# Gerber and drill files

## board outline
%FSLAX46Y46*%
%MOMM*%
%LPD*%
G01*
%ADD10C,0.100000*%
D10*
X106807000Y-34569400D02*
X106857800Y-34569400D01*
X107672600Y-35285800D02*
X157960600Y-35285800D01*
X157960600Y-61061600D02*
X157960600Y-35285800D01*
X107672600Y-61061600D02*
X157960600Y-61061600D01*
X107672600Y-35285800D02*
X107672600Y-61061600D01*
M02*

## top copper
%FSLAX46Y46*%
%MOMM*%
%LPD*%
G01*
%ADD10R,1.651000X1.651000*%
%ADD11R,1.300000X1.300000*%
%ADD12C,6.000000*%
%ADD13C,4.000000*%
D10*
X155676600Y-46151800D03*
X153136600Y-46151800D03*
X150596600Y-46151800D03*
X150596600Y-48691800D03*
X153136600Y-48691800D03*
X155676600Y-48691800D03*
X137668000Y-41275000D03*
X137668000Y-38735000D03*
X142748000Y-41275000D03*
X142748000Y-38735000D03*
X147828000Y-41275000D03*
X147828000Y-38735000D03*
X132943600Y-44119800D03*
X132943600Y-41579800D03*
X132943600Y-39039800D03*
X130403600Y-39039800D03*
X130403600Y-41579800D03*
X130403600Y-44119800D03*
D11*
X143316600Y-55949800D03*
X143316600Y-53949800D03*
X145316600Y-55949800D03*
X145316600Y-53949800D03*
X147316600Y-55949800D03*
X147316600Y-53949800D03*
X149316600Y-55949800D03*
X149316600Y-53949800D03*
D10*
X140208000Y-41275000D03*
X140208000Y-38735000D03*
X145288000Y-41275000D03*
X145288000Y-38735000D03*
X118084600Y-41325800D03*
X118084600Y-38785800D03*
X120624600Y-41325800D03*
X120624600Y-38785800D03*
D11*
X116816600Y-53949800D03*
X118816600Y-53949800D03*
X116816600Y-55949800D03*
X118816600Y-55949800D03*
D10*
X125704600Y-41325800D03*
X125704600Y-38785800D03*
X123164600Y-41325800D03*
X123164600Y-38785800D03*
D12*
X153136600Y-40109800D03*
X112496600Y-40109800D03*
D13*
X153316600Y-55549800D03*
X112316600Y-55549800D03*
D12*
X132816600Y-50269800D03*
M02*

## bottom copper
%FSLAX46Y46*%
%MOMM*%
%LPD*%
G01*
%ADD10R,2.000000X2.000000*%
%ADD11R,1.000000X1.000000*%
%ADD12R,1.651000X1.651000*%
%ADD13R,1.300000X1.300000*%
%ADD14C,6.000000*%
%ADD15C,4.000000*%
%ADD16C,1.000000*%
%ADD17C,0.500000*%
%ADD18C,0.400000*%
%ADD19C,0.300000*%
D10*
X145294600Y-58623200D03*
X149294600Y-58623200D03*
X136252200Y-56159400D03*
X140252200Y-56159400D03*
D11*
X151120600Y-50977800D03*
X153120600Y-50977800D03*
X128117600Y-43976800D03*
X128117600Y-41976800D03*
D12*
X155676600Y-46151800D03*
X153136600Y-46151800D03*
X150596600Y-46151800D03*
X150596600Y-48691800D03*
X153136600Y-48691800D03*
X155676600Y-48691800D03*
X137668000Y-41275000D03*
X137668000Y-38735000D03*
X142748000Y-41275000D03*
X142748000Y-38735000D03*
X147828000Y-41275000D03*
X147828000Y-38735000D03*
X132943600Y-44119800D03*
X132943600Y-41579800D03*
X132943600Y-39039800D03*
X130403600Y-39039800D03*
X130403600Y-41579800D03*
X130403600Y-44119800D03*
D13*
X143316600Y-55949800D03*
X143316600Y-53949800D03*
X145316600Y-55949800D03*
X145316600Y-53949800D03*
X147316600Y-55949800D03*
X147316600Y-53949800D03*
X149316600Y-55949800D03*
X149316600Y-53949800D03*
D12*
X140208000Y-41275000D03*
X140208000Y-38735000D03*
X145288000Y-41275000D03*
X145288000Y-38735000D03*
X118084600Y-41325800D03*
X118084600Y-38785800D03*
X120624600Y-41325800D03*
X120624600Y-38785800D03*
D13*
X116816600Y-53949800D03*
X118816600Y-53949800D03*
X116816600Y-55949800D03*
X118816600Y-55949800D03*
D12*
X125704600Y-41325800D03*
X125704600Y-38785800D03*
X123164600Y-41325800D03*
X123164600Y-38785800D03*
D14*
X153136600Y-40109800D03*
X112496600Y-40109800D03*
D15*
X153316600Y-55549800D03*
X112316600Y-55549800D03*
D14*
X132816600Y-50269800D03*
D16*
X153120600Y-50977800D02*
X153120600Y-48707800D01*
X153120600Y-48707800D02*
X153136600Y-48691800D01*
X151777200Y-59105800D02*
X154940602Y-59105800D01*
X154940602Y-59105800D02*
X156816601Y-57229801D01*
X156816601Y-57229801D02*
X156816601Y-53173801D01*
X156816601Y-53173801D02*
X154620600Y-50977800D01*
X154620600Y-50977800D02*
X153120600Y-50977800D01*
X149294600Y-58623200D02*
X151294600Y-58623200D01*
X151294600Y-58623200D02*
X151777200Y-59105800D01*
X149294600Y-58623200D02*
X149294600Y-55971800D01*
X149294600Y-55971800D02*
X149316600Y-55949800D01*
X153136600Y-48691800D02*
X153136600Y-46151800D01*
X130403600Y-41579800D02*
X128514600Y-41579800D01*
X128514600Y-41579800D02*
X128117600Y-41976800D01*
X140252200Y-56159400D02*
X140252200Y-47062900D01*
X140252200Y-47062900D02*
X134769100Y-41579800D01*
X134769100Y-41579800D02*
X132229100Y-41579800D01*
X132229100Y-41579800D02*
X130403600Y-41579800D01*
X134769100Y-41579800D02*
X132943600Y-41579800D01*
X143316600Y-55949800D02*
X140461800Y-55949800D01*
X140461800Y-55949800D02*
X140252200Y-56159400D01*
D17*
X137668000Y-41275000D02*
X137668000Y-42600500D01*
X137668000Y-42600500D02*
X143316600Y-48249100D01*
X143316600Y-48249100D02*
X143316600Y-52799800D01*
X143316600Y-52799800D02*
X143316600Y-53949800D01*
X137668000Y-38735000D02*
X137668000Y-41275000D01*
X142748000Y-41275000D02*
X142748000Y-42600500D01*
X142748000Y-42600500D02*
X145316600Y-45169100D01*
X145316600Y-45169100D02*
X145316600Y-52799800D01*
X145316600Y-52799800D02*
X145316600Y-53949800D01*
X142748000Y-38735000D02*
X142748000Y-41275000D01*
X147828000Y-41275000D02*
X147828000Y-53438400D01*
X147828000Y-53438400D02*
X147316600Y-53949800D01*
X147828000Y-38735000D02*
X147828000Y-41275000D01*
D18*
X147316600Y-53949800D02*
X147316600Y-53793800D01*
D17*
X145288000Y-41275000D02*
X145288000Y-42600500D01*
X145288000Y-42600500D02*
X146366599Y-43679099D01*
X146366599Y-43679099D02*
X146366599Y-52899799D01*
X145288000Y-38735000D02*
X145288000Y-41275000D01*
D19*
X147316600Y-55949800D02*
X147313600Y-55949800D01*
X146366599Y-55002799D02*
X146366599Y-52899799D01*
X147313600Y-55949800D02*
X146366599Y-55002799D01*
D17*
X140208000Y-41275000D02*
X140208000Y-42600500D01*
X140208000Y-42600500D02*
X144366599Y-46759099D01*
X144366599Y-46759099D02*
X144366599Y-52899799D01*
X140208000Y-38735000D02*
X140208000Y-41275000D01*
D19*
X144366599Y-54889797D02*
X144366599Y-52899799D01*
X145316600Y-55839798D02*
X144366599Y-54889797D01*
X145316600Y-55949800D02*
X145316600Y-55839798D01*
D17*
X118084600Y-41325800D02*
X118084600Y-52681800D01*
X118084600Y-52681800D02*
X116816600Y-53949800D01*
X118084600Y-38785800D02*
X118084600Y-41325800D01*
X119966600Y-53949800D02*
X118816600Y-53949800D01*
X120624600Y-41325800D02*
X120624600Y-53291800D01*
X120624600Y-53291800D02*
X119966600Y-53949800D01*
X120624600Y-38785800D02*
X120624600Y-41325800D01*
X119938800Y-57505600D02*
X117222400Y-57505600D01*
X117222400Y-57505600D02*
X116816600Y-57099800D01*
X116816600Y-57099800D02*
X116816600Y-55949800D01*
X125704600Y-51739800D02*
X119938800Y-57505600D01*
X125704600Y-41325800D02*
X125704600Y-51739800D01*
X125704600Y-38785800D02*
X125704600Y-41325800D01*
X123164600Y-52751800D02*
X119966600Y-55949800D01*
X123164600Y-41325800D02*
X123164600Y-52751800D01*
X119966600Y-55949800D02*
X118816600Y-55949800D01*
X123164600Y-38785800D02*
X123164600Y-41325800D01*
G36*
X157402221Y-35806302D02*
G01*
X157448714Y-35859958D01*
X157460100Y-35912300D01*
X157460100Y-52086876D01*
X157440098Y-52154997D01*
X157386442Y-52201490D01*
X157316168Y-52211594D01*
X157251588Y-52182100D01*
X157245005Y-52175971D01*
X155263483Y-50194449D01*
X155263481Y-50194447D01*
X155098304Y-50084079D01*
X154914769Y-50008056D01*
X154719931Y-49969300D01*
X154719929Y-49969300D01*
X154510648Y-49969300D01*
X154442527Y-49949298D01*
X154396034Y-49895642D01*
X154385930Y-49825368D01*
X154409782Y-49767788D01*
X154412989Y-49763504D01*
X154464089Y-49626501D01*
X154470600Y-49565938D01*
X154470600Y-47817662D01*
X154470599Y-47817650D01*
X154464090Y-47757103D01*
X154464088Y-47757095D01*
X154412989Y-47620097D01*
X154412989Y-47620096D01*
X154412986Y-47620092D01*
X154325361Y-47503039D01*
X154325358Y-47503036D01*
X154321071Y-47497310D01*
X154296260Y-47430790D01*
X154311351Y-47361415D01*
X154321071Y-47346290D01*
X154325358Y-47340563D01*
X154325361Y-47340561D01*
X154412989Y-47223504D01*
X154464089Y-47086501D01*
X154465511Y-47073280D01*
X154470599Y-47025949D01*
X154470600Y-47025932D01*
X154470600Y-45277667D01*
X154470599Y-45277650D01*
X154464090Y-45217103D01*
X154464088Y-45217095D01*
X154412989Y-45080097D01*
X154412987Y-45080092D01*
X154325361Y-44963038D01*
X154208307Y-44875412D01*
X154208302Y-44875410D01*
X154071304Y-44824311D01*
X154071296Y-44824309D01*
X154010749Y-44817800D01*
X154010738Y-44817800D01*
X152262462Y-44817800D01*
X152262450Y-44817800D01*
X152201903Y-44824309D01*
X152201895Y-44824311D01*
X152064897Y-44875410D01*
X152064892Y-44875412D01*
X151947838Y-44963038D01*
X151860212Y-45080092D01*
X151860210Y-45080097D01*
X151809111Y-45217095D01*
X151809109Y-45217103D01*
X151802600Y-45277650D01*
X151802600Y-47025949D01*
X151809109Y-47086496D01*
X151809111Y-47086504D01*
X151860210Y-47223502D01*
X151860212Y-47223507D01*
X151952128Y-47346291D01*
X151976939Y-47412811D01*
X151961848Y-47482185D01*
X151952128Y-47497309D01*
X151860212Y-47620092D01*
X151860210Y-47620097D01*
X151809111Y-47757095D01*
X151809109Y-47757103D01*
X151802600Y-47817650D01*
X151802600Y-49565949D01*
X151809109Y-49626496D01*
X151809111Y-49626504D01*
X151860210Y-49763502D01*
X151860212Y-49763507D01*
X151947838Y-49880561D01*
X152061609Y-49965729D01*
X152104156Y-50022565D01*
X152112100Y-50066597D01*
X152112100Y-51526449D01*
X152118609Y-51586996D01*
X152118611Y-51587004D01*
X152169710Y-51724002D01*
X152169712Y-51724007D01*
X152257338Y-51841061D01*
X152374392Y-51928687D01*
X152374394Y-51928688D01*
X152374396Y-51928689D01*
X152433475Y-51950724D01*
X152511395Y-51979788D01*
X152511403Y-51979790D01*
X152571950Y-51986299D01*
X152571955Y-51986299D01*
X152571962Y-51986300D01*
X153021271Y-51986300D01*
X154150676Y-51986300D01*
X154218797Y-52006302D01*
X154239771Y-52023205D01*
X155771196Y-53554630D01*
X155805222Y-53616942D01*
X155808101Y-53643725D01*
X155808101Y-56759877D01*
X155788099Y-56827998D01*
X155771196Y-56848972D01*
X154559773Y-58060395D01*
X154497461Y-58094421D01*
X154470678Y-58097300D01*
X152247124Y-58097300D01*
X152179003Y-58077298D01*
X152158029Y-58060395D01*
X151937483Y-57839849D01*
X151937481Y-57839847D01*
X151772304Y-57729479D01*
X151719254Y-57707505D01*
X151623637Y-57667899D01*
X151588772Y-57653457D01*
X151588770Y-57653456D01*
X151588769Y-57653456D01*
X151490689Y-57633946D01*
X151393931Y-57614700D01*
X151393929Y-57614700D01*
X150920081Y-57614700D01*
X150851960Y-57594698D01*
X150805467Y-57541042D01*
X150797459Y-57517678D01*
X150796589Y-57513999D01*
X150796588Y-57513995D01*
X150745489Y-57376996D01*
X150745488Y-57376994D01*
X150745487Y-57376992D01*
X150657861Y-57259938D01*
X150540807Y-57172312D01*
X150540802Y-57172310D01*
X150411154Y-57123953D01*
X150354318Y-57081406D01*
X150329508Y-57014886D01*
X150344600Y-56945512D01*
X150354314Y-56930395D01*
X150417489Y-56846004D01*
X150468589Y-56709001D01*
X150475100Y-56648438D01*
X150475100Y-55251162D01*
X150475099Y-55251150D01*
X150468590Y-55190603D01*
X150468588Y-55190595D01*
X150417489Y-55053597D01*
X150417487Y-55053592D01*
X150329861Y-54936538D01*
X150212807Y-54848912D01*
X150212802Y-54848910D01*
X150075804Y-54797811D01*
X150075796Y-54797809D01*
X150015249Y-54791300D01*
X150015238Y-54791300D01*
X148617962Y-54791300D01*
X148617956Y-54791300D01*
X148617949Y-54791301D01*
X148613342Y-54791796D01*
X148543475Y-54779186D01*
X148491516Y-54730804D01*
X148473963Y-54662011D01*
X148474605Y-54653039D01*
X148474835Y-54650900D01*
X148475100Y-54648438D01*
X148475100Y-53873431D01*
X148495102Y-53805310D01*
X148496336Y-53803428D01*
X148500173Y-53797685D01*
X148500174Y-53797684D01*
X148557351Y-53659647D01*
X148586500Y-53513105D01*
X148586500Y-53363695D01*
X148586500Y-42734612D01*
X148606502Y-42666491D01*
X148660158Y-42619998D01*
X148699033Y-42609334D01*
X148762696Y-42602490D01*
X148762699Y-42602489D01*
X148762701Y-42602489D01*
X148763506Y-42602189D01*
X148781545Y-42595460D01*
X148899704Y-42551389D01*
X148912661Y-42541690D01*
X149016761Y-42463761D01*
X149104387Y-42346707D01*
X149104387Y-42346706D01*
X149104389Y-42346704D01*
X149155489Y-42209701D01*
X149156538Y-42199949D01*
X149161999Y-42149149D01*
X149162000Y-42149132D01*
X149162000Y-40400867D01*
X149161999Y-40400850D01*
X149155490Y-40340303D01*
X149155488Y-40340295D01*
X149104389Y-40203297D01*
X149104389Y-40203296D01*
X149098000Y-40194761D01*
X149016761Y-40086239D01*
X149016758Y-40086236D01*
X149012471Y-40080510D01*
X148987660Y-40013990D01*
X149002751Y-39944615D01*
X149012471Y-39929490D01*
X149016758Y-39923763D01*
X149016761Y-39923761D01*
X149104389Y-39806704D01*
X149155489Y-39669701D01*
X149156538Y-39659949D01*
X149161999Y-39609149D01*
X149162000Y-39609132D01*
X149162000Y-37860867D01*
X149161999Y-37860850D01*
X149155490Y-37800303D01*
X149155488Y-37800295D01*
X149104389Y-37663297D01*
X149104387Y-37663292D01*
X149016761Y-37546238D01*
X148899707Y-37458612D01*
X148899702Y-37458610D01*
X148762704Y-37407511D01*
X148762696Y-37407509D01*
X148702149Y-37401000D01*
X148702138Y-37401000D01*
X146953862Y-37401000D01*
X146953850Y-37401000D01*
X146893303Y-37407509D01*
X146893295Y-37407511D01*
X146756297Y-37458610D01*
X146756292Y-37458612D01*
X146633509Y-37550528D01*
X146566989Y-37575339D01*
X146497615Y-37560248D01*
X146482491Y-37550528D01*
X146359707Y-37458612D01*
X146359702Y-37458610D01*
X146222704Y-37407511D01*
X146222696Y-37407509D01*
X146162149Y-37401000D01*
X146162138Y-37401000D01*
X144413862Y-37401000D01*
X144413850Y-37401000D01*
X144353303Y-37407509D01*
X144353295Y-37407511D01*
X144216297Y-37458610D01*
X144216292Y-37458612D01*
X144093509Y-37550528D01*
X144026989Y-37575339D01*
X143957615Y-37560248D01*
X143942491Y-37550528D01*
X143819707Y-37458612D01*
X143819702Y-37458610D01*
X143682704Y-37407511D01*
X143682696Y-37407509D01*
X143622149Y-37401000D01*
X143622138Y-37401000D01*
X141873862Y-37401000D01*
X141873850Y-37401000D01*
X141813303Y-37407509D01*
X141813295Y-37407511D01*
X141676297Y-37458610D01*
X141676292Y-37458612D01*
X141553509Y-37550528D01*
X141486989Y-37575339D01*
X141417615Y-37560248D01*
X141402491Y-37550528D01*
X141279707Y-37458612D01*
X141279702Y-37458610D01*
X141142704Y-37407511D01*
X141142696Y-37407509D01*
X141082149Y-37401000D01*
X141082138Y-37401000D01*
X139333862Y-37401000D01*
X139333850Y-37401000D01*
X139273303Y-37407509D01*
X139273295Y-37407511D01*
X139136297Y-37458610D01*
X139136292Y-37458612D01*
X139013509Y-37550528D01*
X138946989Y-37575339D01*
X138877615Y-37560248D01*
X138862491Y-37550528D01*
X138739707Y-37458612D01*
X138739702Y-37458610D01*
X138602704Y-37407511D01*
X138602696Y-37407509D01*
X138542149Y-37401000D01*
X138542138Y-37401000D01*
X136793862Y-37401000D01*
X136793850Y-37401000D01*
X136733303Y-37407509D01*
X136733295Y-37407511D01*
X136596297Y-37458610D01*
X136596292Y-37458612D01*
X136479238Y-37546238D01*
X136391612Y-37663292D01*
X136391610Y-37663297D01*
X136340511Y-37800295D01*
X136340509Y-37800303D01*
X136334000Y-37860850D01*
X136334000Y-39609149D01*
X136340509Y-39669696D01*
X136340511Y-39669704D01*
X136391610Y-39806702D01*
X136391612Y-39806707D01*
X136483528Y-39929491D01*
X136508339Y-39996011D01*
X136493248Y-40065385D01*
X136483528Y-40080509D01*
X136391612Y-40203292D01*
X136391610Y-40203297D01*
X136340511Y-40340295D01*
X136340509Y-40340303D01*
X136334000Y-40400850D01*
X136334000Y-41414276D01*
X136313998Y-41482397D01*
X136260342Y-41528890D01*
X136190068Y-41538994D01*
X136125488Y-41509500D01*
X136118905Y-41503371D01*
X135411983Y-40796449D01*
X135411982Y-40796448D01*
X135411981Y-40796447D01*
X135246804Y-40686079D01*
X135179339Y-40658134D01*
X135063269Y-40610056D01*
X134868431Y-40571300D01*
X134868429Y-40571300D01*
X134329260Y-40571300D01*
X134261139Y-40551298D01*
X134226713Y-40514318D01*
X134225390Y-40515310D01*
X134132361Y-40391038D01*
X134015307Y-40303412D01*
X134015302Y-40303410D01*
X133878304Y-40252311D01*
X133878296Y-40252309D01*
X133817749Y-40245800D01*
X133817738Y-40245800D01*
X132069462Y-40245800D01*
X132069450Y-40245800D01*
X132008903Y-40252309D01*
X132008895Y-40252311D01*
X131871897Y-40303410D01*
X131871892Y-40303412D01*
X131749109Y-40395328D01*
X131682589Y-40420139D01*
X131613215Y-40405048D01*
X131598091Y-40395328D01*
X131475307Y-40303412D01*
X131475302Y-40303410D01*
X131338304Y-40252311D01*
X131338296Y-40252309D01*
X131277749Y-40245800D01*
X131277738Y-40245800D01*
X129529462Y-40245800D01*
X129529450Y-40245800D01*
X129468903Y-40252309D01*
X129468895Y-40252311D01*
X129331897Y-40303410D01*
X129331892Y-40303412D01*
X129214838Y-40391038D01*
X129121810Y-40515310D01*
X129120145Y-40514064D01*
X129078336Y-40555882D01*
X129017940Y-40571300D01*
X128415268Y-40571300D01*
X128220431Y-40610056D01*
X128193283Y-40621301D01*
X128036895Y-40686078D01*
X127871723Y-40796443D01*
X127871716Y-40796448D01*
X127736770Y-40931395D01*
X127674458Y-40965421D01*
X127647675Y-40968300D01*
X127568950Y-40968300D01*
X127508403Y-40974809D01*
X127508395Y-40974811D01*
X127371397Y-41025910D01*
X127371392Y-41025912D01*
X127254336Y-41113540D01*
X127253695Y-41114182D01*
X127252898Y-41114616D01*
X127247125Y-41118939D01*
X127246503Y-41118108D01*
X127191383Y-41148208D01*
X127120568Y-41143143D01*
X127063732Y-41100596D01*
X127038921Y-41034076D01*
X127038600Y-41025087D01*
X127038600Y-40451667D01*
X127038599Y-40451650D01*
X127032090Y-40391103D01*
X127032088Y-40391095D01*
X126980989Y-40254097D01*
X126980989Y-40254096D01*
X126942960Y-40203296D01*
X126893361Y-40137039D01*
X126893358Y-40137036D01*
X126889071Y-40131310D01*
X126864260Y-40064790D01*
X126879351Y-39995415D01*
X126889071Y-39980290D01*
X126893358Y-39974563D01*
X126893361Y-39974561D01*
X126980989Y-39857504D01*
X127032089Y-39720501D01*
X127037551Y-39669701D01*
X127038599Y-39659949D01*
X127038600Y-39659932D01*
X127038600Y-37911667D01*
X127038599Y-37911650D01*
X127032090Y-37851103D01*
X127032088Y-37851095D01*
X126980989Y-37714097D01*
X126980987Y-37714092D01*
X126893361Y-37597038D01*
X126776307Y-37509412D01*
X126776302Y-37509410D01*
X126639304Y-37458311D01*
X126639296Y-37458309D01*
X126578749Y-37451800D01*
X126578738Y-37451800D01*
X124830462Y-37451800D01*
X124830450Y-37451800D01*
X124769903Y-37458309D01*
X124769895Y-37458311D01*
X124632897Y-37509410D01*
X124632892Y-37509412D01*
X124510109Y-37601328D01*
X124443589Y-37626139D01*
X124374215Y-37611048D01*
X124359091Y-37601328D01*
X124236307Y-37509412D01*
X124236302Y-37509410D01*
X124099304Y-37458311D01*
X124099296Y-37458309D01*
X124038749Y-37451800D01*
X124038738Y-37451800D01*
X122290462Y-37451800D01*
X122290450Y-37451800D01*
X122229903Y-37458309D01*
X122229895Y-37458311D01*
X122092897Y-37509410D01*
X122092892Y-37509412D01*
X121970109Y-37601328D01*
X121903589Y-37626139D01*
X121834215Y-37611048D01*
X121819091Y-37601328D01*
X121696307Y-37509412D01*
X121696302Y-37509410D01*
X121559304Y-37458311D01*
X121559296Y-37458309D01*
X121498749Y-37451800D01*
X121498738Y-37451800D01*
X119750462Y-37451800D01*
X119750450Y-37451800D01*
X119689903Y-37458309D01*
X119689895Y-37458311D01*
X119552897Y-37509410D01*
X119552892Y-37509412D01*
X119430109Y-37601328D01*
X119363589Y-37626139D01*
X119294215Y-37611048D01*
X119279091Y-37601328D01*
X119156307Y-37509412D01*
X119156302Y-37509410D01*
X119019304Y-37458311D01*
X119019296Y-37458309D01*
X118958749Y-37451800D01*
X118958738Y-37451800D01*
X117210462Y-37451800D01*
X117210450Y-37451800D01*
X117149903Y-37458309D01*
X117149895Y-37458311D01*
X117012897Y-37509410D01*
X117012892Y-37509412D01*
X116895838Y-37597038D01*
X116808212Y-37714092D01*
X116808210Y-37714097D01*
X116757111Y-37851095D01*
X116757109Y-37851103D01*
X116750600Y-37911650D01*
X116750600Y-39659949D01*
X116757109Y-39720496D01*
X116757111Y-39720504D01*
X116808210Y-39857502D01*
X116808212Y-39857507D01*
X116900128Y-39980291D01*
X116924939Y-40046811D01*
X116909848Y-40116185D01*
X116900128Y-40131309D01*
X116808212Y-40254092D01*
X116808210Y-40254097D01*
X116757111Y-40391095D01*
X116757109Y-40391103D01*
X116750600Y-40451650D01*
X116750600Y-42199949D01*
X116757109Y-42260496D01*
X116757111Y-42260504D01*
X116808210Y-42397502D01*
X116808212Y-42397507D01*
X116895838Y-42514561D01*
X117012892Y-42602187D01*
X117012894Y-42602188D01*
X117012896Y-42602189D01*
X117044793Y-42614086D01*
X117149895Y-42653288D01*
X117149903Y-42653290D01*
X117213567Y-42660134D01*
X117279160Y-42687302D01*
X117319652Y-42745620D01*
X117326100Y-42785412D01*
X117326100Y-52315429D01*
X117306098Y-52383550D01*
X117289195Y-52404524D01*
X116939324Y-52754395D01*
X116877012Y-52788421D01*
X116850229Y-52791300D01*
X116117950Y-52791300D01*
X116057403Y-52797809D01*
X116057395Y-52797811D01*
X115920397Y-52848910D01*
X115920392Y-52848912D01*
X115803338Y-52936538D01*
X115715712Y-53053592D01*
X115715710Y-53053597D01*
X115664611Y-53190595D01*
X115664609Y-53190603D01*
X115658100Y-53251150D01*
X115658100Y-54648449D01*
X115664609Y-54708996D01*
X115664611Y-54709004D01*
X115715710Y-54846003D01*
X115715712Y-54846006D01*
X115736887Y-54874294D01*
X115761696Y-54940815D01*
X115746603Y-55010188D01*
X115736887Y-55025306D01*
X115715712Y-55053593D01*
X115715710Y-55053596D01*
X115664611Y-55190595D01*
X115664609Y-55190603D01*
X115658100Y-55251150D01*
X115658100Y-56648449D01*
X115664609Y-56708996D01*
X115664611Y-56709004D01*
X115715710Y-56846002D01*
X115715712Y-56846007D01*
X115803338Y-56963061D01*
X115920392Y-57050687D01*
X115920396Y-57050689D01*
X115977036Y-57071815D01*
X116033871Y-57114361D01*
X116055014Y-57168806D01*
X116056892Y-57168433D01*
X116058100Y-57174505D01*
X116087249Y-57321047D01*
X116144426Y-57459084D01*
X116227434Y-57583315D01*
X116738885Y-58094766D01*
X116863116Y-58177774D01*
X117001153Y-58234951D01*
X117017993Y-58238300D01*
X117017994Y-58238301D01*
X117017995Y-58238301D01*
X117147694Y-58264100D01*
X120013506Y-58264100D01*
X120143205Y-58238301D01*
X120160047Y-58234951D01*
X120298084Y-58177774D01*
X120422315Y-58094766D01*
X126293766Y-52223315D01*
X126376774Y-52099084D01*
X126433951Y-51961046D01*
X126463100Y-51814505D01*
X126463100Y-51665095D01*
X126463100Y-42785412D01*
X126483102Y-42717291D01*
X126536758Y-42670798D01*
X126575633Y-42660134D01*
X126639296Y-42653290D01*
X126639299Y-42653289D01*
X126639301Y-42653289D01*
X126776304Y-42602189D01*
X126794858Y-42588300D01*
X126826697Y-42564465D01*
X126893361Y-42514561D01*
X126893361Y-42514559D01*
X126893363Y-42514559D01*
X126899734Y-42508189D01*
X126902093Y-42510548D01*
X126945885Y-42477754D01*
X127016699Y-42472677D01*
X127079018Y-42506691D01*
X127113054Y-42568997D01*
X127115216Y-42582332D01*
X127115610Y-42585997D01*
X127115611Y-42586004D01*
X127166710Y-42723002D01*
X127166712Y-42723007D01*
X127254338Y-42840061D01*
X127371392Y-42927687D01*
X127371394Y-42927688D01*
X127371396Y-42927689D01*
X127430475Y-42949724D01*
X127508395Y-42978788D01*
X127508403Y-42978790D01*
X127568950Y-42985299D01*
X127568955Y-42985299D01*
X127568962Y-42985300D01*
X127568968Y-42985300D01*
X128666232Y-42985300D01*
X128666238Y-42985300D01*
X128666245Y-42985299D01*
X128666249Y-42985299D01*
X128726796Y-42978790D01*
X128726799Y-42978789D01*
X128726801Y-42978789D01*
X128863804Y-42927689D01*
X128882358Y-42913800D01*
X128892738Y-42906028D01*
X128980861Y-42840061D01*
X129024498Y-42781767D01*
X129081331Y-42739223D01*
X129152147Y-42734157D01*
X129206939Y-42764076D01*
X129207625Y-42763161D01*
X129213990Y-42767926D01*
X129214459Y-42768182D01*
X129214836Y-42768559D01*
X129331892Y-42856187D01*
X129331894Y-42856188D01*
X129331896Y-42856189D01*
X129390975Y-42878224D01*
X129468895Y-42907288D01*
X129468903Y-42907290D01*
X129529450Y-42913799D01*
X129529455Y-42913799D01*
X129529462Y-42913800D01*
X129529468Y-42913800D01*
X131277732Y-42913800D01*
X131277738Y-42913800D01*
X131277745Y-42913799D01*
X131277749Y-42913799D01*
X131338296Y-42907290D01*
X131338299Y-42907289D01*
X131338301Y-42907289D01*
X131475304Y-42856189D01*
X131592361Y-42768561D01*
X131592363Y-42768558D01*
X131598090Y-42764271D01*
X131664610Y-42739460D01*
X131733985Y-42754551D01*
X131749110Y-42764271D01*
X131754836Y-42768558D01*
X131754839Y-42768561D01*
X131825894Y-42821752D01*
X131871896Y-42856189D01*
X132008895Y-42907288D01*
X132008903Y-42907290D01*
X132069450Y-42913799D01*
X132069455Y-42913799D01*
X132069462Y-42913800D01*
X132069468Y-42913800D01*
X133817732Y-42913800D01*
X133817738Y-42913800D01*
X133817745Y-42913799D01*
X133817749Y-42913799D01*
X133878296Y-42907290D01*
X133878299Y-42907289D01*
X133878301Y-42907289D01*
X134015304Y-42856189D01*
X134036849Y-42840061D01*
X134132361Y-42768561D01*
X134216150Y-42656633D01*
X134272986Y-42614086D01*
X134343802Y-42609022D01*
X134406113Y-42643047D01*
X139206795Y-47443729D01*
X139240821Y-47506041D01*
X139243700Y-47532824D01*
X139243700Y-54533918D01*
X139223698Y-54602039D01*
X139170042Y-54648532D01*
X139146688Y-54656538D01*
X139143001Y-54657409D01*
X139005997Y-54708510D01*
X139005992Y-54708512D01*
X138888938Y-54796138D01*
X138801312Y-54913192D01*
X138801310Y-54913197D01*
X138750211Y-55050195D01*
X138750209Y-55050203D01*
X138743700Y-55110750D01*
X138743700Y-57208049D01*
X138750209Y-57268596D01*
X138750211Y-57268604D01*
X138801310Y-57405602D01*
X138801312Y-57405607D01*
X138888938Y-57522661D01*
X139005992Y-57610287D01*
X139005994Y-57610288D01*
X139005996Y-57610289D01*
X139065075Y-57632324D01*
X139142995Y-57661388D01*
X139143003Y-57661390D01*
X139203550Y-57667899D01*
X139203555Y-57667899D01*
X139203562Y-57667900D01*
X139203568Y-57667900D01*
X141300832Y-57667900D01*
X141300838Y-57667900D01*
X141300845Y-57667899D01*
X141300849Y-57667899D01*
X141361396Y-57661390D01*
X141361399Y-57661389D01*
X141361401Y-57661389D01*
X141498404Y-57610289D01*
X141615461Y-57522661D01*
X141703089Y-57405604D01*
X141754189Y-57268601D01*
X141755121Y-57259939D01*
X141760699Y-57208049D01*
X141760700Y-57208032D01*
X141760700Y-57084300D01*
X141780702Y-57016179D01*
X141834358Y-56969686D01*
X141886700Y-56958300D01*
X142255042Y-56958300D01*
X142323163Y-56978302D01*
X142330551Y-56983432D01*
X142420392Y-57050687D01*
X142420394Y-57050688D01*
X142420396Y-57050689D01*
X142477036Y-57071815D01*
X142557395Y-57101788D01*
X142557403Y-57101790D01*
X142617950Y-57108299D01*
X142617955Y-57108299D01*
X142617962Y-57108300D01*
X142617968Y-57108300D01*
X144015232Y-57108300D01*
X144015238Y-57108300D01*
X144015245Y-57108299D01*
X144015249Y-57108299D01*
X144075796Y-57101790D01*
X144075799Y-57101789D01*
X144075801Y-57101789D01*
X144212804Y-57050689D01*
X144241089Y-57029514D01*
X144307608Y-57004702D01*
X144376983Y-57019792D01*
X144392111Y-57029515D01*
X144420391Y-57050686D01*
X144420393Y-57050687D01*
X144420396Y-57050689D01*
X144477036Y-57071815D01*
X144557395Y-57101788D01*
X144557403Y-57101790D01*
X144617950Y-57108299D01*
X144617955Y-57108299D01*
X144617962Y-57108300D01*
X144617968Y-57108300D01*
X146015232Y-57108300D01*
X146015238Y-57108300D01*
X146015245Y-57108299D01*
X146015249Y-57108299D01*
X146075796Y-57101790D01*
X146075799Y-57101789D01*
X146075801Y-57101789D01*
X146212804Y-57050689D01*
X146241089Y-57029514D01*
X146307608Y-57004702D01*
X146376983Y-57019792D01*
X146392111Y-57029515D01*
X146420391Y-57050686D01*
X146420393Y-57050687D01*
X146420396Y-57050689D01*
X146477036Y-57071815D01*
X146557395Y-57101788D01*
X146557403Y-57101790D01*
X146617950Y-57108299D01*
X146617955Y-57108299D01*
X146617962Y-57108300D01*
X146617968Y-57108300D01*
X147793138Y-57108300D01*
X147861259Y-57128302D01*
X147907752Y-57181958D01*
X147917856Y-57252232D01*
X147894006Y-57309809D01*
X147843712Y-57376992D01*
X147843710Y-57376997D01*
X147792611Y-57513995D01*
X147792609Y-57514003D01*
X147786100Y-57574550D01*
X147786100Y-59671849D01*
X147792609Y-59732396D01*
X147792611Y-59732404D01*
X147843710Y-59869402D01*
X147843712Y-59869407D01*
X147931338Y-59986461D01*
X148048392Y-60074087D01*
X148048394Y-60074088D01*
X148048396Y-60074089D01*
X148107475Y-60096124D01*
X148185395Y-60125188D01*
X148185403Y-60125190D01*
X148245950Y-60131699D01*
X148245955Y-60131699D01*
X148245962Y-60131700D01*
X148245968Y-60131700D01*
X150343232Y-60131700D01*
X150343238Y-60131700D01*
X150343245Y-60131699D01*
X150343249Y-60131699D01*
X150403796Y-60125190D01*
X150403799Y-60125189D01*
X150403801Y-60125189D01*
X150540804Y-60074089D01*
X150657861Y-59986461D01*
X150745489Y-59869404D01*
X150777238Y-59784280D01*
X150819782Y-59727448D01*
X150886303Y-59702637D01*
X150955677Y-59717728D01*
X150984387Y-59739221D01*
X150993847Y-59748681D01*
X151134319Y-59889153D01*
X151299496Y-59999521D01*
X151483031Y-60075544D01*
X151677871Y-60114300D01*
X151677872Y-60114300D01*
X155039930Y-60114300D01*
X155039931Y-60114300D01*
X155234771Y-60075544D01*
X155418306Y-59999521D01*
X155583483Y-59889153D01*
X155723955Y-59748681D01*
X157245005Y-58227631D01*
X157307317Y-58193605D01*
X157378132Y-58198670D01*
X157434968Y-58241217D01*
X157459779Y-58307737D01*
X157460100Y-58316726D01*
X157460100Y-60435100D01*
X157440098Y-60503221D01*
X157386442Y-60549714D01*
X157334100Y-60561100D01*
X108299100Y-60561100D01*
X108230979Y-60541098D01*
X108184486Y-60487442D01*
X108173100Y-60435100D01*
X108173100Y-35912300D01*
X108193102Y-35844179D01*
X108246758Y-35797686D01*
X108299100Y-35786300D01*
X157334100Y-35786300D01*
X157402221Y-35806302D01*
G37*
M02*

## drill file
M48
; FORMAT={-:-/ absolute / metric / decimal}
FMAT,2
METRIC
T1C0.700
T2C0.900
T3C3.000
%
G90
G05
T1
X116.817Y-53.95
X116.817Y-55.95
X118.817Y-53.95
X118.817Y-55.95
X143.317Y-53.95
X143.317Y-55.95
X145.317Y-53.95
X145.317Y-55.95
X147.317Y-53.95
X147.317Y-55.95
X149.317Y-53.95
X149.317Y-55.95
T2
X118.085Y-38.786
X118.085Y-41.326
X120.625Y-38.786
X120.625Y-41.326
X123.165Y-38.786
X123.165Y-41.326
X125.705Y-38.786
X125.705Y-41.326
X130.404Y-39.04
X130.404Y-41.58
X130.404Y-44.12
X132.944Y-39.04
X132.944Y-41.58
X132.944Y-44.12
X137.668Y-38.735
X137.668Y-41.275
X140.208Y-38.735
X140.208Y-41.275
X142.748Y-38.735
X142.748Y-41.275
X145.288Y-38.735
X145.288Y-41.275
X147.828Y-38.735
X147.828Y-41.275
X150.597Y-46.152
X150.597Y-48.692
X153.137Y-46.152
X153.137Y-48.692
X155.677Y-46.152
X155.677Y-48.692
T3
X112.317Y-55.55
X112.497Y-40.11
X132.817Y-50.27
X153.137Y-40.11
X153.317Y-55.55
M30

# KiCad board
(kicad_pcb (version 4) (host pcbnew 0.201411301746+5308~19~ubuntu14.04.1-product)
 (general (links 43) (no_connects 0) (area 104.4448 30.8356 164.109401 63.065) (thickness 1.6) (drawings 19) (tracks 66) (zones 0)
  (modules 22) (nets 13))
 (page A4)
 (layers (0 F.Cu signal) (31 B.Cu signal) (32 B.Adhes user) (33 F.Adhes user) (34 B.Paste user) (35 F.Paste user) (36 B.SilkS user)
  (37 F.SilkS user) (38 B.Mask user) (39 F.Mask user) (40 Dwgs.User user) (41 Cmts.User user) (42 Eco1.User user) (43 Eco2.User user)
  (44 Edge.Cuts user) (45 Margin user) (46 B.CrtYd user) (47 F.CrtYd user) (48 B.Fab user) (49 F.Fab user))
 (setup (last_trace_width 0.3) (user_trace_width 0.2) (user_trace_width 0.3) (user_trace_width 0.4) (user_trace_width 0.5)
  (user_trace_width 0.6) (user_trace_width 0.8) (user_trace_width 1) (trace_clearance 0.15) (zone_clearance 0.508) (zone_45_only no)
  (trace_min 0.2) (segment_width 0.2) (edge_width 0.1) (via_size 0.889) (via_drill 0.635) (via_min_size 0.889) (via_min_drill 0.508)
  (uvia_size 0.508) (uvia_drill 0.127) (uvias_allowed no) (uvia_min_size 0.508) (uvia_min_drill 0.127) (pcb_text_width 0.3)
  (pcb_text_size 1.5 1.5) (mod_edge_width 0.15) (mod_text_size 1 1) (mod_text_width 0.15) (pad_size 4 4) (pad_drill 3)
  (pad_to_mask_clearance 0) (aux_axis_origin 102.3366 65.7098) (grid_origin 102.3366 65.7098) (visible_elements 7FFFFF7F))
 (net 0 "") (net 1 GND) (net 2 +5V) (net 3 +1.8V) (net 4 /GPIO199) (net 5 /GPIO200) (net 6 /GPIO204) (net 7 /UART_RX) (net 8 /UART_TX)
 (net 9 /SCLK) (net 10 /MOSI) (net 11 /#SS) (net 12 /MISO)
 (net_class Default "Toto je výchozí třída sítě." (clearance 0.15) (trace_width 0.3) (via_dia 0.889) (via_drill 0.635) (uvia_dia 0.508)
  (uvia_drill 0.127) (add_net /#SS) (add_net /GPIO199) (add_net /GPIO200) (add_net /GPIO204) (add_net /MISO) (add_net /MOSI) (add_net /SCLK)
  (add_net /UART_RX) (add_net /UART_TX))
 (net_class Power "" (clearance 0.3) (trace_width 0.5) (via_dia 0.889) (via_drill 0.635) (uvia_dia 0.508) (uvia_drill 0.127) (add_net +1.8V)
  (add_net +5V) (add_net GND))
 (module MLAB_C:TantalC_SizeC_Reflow (layer B.Cu) (at 147.2946 58.6232 180)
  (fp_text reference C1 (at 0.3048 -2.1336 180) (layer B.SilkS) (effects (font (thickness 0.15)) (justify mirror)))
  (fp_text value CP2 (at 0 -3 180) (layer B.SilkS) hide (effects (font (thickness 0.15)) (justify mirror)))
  (pad 2 smd rect (at 2 0 180) (size 2 2) (layers B.Cu B.Paste B.Mask) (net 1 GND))
  (pad 1 smd rect (at -2 0 180) (size 2 2) (layers B.Cu B.Paste B.Mask) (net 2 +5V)))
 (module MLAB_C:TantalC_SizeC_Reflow (layer B.Cu) (at 138.2522 56.1594 180)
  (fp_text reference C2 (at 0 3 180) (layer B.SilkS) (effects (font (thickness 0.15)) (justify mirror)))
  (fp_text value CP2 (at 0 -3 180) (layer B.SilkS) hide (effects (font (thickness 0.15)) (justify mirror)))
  (pad 2 smd rect (at 2 0 180) (size 2 2) (layers B.Cu B.Paste B.Mask) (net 1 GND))
  (pad 1 smd rect (at -2 0 180) (size 2 2) (layers B.Cu B.Paste B.Mask) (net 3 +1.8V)))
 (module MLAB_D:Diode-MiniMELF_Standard (layer B.Cu) (at 152.1206 50.9778)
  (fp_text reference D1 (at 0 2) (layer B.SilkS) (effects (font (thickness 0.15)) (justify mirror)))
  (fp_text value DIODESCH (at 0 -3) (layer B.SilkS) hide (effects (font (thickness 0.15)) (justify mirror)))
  (pad 1 smd rect (at -1 0) (size 1 1) (layers B.Cu B.Paste B.Mask) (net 1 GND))
  (pad 2 smd rect (at 1 0) (size 1 1) (layers B.Cu B.Paste B.Mask) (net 2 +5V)))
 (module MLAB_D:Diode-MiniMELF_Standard (layer B.Cu) (at 128.1176 42.9768 90)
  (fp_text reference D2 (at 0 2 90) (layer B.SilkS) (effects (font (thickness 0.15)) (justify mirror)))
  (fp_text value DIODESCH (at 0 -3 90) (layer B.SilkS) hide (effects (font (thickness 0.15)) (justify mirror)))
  (pad 1 smd rect (at -1 0 90) (size 1 1) (layers B.Cu B.Paste B.Mask) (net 1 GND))
  (pad 2 smd rect (at 1 0 90) (size 1 1) (layers B.Cu B.Paste B.Mask) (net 3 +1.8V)))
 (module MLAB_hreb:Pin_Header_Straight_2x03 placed (layer F.Cu) (at 153.1366 47.4218 180)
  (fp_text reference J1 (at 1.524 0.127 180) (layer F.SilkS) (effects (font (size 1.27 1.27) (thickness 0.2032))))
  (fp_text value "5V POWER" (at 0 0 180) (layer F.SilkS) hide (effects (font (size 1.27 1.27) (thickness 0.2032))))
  (pad 1 thru_hole rect (at -2.54 1.27 180) (size 1.651 1.651) (drill 0.9) (layers *.Cu *.Mask F.SilkS) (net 1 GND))
  (pad 2 thru_hole rect (at 0 1.27 180) (size 1.651 1.651) (drill 0.9) (layers *.Cu *.Mask F.SilkS) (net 2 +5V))
  (pad 3 thru_hole rect (at 2.54 1.27 180) (size 1.651 1.651) (drill 0.9) (layers *.Cu *.Mask F.SilkS) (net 1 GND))
  (pad 4 thru_hole rect (at 2.54 -1.27 180) (size 1.651 1.651) (drill 0.9) (layers *.Cu *.Mask F.SilkS) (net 1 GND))
  (pad 5 thru_hole rect (at 0 -1.27 180) (size 1.651 1.651) (drill 0.9) (layers *.Cu *.Mask F.SilkS) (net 2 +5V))
  (pad 6 thru_hole rect (at -2.54 -1.27 180) (size 1.651 1.651) (drill 0.9) (layers *.Cu *.Mask F.SilkS) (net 1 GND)))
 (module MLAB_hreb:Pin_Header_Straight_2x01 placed (layer F.Cu) (at 137.668 40.005)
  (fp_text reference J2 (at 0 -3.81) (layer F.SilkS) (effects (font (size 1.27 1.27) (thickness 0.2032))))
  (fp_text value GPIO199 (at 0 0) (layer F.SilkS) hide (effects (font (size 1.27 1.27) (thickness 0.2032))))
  (pad 2 thru_hole rect (at 0 1.27) (size 1.651 1.651) (drill 0.9) (layers *.Cu *.Mask F.SilkS) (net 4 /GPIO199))
  (pad 1 thru_hole rect (at 0 -1.27) (size 1.651 1.651) (drill 0.9) (layers *.Cu *.Mask F.SilkS) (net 4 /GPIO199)))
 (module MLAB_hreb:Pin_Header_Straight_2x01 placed (layer F.Cu) (at 142.748 40.005)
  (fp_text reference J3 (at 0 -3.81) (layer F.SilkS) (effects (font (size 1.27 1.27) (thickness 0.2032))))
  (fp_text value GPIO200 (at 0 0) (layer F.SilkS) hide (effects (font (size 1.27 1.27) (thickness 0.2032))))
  (pad 2 thru_hole rect (at 0 1.27) (size 1.651 1.651) (drill 0.9) (layers *.Cu *.Mask F.SilkS) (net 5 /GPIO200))
  (pad 1 thru_hole rect (at 0 -1.27) (size 1.651 1.651) (drill 0.9) (layers *.Cu *.Mask F.SilkS) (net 5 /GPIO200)))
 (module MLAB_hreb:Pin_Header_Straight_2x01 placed (layer F.Cu) (at 147.828 40.005)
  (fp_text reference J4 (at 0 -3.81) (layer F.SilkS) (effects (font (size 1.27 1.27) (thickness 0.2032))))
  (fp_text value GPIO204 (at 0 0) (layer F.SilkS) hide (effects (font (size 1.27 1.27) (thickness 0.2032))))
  (pad 2 thru_hole rect (at 0 1.27) (size 1.651 1.651) (drill 0.9) (layers *.Cu *.Mask F.SilkS) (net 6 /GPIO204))
  (pad 1 thru_hole rect (at 0 -1.27) (size 1.651 1.651) (drill 0.9) (layers *.Cu *.Mask F.SilkS) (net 6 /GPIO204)))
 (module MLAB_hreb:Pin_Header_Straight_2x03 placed (layer F.Cu) (at 131.6736 41.5798 90)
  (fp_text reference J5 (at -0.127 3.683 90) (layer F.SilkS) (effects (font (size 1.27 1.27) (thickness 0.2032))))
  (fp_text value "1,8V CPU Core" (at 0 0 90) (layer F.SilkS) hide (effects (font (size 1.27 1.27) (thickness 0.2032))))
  (pad 1 thru_hole rect (at -2.54 1.27 90) (size 1.651 1.651) (drill 0.9) (layers *.Cu *.Mask F.SilkS) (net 1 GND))
  (pad 2 thru_hole rect (at 0 1.27 90) (size 1.651 1.651) (drill 0.9) (layers *.Cu *.Mask F.SilkS) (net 3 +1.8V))
  (pad 3 thru_hole rect (at 2.54 1.27 90) (size 1.651 1.651) (drill 0.9) (layers *.Cu *.Mask F.SilkS) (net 1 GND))
  (pad 4 thru_hole rect (at 2.54 -1.27 90) (size 1.651 1.651) (drill 0.9) (layers *.Cu *.Mask F.SilkS) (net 1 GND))
  (pad 5 thru_hole rect (at 0 -1.27 90) (size 1.651 1.651) (drill 0.9) (layers *.Cu *.Mask F.SilkS) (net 3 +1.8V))
  (pad 6 thru_hole rect (at -2.54 -1.27 90) (size 1.651 1.651) (drill 0.9) (layers *.Cu *.Mask F.SilkS) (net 1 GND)))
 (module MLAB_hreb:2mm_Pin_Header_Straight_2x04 (layer F.Cu) (at 146.3166 54.9498 90)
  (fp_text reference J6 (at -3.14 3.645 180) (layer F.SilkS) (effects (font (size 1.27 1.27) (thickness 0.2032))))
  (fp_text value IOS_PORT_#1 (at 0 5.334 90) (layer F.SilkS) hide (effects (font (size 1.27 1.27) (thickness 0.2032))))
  (pad 1 thru_hole rect (at -1 -3 90) (size 1.3 1.3) (drill 0.7) (layers *.Cu *.Mask F.SilkS) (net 3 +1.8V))
  (pad 2 thru_hole rect (at 1 -3 90) (size 1.3 1.3) (drill 0.7) (layers *.Cu *.Mask F.SilkS) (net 4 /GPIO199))
  (pad 3 thru_hole rect (at -1 -1 90) (size 1.3 1.3) (drill 0.7) (layers *.Cu *.Mask F.SilkS) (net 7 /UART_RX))
  (pad 4 thru_hole rect (at 1 -1 90) (size 1.3 1.3) (drill 0.7) (layers *.Cu *.Mask F.SilkS) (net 5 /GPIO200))
  (pad 5 thru_hole rect (at -1 1 90) (size 1.3 1.3) (drill 0.7) (layers *.Cu *.Mask F.SilkS) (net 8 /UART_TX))
  (pad 6 thru_hole rect (at 1 1 90) (size 1.3 1.3) (drill 0.7) (layers *.Cu *.Mask F.SilkS) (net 6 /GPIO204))
  (pad 7 thru_hole rect (at -1 3 90) (size 1.3 1.3) (drill 0.7) (layers *.Cu *.Mask F.SilkS) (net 2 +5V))
  (pad 8 thru_hole rect (at 1 3 90) (size 1.3 1.3) (drill 0.7) (layers *.Cu *.Mask F.SilkS) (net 1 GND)))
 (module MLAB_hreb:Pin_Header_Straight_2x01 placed (layer F.Cu) (at 140.208 40.005)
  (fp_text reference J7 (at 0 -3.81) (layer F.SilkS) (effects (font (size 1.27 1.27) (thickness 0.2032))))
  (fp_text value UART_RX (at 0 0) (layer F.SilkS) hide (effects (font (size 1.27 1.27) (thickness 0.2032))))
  (pad 2 thru_hole rect (at 0 1.27) (size 1.651 1.651) (drill 0.9) (layers *.Cu *.Mask F.SilkS) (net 7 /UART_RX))
  (pad 1 thru_hole rect (at 0 -1.27) (size 1.651 1.651) (drill 0.9) (layers *.Cu *.Mask F.SilkS) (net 7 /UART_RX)))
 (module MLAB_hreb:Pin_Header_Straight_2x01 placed (layer F.Cu) (at 145.288 40.005)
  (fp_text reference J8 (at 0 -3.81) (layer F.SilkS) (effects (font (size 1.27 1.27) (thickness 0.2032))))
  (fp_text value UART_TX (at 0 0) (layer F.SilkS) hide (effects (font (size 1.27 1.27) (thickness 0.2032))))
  (pad 2 thru_hole rect (at 0 1.27) (size 1.651 1.651) (drill 0.9) (layers *.Cu *.Mask F.SilkS) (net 8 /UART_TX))
  (pad 1 thru_hole rect (at 0 -1.27) (size 1.651 1.651) (drill 0.9) (layers *.Cu *.Mask F.SilkS) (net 8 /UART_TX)))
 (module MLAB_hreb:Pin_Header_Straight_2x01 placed (layer F.Cu) (at 118.0846 40.0558)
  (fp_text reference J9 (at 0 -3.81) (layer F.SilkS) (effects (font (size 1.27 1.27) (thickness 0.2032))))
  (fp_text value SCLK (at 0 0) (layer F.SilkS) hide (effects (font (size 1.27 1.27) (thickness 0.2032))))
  (pad 2 thru_hole rect (at 0 1.27) (size 1.651 1.651) (drill 0.9) (layers *.Cu *.Mask F.SilkS) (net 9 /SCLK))
  (pad 1 thru_hole rect (at 0 -1.27) (size 1.651 1.651) (drill 0.9) (layers *.Cu *.Mask F.SilkS) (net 9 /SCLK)))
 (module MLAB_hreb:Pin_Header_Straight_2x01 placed (layer F.Cu) (at 120.6246 40.0558)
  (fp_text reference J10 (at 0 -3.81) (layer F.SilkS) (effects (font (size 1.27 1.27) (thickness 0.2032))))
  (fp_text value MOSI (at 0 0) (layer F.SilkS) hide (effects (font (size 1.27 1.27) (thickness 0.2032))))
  (pad 2 thru_hole rect (at 0 1.27) (size 1.651 1.651) (drill 0.9) (layers *.Cu *.Mask F.SilkS) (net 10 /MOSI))
  (pad 1 thru_hole rect (at 0 -1.27) (size 1.651 1.651) (drill 0.9) (layers *.Cu *.Mask F.SilkS) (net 10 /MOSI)))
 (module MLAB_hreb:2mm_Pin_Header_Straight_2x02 (layer F.Cu) (at 117.8166 54.9498)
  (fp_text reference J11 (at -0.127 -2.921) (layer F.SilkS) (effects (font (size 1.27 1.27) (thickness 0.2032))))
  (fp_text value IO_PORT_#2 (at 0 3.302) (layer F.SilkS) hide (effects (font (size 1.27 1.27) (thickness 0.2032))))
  (pad 1 thru_hole rect (at -1 -1) (size 1.3 1.3) (drill 0.7) (layers *.Cu *.Mask F.SilkS) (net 9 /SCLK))
  (pad 2 thru_hole rect (at 1 -1) (size 1.3 1.3) (drill 0.7) (layers *.Cu *.Mask F.SilkS) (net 10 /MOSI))
  (pad 3 thru_hole rect (at -1 1) (size 1.3 1.3) (drill 0.7) (layers *.Cu *.Mask F.SilkS) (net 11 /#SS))
  (pad 4 thru_hole rect (at 1 1) (size 1.3 1.3) (drill 0.7) (layers *.Cu *.Mask F.SilkS) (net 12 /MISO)))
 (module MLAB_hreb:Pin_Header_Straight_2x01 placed (layer F.Cu) (at 125.7046 40.0558)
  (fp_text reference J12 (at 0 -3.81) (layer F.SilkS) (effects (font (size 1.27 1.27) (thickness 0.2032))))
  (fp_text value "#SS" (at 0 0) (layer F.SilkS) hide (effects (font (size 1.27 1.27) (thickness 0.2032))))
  (pad 2 thru_hole rect (at 0 1.27) (size 1.651 1.651) (drill 0.9) (layers *.Cu *.Mask F.SilkS) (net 11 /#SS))
  (pad 1 thru_hole rect (at 0 -1.27) (size 1.651 1.651) (drill 0.9) (layers *.Cu *.Mask F.SilkS) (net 11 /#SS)))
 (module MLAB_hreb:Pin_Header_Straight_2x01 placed (layer F.Cu) (at 123.1646 40.0558)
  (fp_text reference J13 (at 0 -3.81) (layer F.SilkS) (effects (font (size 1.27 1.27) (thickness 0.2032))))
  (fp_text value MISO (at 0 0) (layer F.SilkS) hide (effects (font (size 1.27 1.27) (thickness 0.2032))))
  (pad 2 thru_hole rect (at 0 1.27) (size 1.651 1.651) (drill 0.9) (layers *.Cu *.Mask F.SilkS) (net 12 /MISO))
  (pad 1 thru_hole rect (at 0 -1.27) (size 1.651 1.651) (drill 0.9) (layers *.Cu *.Mask F.SilkS) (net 12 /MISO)))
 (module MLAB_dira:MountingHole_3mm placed (layer F.Cu) (at 153.1366 40.1098)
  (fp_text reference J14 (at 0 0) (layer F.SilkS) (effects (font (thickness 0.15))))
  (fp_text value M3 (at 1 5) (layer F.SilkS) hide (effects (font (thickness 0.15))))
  (pad 1 thru_hole circle (at 0 0) (size 6 6) (drill 3) (layers *.Cu *.Adhes *.Mask) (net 1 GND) (clearance 1) (zone_connect 2)))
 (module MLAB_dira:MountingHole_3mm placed (layer F.Cu) (at 112.4966 40.1098)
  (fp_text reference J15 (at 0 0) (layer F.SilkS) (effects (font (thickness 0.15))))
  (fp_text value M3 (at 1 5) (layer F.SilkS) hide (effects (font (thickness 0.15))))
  (pad 1 thru_hole circle (at 0 0) (size 6 6) (drill 3) (layers *.Cu *.Adhes *.Mask) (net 1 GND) (clearance 1) (zone_connect 2)))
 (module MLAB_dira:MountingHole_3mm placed (layer F.Cu) (at 153.3166 55.5498)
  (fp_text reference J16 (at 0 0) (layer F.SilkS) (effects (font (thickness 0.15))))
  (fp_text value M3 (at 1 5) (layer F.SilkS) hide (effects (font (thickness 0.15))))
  (pad 1 thru_hole circle (at 0 0) (size 4 4) (drill 3) (layers *.Cu *.Adhes *.Mask) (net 1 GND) (clearance 1) (zone_connect 2)))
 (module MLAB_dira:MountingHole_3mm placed (layer F.Cu) (at 112.3166 55.5498)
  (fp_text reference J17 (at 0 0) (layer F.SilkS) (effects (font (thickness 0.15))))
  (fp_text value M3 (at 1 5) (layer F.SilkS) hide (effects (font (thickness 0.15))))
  (pad 1 thru_hole circle (at 0 0) (size 4 4) (drill 3) (layers *.Cu *.Adhes *.Mask) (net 1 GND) (clearance 1) (zone_connect 2)))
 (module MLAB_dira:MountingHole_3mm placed (layer F.Cu) (at 132.8166 50.2698)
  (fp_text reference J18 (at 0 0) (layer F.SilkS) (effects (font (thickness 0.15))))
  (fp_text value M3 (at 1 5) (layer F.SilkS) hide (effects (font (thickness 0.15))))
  (pad 1 thru_hole circle (at 0 0) (size 6 6) (drill 3) (layers *.Cu *.Adhes *.Mask) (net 1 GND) (clearance 1) (zone_connect 2)))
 (gr_line (start 106.807 34.5694) (end 106.8578 34.5694) (angle 90) (layer Edge.Cuts) (width 0.1))
 (gr_line (start 107.6726 35.2858) (end 157.9606 35.2858) (angle 90) (layer Edge.Cuts) (width 0.1))
 (gr_line (start 157.9606 61.0616) (end 157.9606 35.2858) (angle 90) (layer Edge.Cuts) (width 0.1))
 (gr_line (start 107.6726 61.0616) (end 157.9606 61.0616) (angle 90) (layer Edge.Cuts) (width 0.1))
 (gr_line (start 107.6726 35.2858) (end 107.6726 61.0616) (angle 90) (layer Edge.Cuts) (width 0.1))
 (segment (start 153.1206 50.9778) (end 153.1206 48.7078) (width 1) (layer B.Cu) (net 2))
 (segment (start 153.1206 48.7078) (end 153.1366 48.6918) (width 1) (layer B.Cu) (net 2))
 (segment (start 151.7772 59.1058) (end 154.940602 59.1058) (width 1) (layer B.Cu) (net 2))
 (segment (start 154.940602 59.1058) (end 156.816601 57.229801) (width 1) (layer B.Cu) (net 2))
 (segment (start 156.816601 57.229801) (end 156.816601 53.173801) (width 1) (layer B.Cu) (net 2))
 (segment (start 156.816601 53.173801) (end 154.6206 50.9778) (width 1) (layer B.Cu) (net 2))
 (segment (start 154.6206 50.9778) (end 153.1206 50.9778) (width 1) (layer B.Cu) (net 2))
 (segment (start 149.2946 58.6232) (end 151.2946 58.6232) (width 1) (layer B.Cu) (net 2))
 (segment (start 151.2946 58.6232) (end 151.7772 59.1058) (width 1) (layer B.Cu) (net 2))
 (segment (start 149.2946 58.6232) (end 149.2946 55.9718) (width 1) (layer B.Cu) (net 2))
 (segment (start 149.2946 55.9718) (end 149.3166 55.9498) (width 1) (layer B.Cu) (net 2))
 (segment (start 153.1366 48.6918) (end 153.1366 46.1518) (width 1) (layer B.Cu) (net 2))
 (segment (start 130.4036 41.5798) (end 128.5146 41.5798) (width 1) (layer B.Cu) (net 3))
 (segment (start 128.5146 41.5798) (end 128.1176 41.9768) (width 1) (layer B.Cu) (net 3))
 (segment (start 140.2522 56.1594) (end 140.2522 47.0629) (width 1) (layer B.Cu) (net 3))
 (segment (start 140.2522 47.0629) (end 134.7691 41.5798) (width 1) (layer B.Cu) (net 3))
 (segment (start 134.7691 41.5798) (end 132.2291 41.5798) (width 1) (layer B.Cu) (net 3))
 (segment (start 132.2291 41.5798) (end 130.4036 41.5798) (width 1) (layer B.Cu) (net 3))
 (segment (start 134.7691 41.5798) (end 132.9436 41.5798) (width 1) (layer B.Cu) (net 3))
 (segment (start 143.3166 55.9498) (end 140.4618 55.9498) (width 1) (layer B.Cu) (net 3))
 (segment (start 140.4618 55.9498) (end 140.2522 56.1594) (width 1) (layer B.Cu) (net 3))
 (segment (start 137.668 41.275) (end 137.668 42.6005) (width 0.5) (layer B.Cu) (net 4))
 (segment (start 137.668 42.6005) (end 143.3166 48.2491) (width 0.5) (layer B.Cu) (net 4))
 (segment (start 143.3166 48.2491) (end 143.3166 52.7998) (width 0.5) (layer B.Cu) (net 4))
 (segment (start 143.3166 52.7998) (end 143.3166 53.9498) (width 0.5) (layer B.Cu) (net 4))
 (segment (start 137.668 38.735) (end 137.668 41.275) (width 0.5) (layer B.Cu) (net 4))
 (segment (start 142.748 41.275) (end 142.748 42.6005) (width 0.5) (layer B.Cu) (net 5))
 (segment (start 142.748 42.6005) (end 145.3166 45.1691) (width 0.5) (layer B.Cu) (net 5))
 (segment (start 145.3166 45.1691) (end 145.3166 52.7998) (width 0.5) (layer B.Cu) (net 5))
 (segment (start 145.3166 52.7998) (end 145.3166 53.9498) (width 0.5) (layer B.Cu) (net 5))
 (segment (start 142.748 38.735) (end 142.748 41.275) (width 0.5) (layer B.Cu) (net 5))
 (segment (start 147.828 41.275) (end 147.828 53.4384) (width 0.5) (layer B.Cu) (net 6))
 (segment (start 147.828 53.4384) (end 147.3166 53.9498) (width 0.5) (layer B.Cu) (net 6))
 (segment (start 147.828 38.735) (end 147.828 41.275) (width 0.5) (layer B.Cu) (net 6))
 (segment (start 147.3166 53.9498) (end 147.3166 53.7938) (width 0.4) (layer B.Cu) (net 6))
 (segment (start 145.288 41.275) (end 145.288 42.6005) (width 0.5) (layer B.Cu) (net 8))
 (segment (start 145.288 42.6005) (end 146.366599 43.679099) (width 0.5) (layer B.Cu) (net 8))
 (segment (start 146.366599 43.679099) (end 146.366599 52.899799) (width 0.5) (layer B.Cu) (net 8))
 (segment (start 145.288 38.735) (end 145.288 41.275) (width 0.5) (layer B.Cu) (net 8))
 (segment (start 147.3166 55.9498) (end 147.3136 55.9498) (width 0.3) (layer B.Cu) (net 8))
 (segment (start 146.366599 55.002799) (end 146.366599 52.899799) (width 0.3) (layer B.Cu) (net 8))
 (segment (start 147.3136 55.9498) (end 146.366599 55.002799) (width 0.3) (layer B.Cu) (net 8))
 (segment (start 140.208 41.275) (end 140.208 42.6005) (width 0.5) (layer B.Cu) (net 7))
 (segment (start 140.208 42.6005) (end 144.366599 46.759099) (width 0.5) (layer B.Cu) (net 7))
 (segment (start 144.366599 46.759099) (end 144.366599 52.899799) (width 0.5) (layer B.Cu) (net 7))
 (segment (start 140.208 38.735) (end 140.208 41.275) (width 0.5) (layer B.Cu) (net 7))
 (segment (start 144.366599 54.889797) (end 144.366599 52.899799) (width 0.3) (layer B.Cu) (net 7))
 (segment (start 145.3166 55.839798) (end 144.366599 54.889797) (width 0.3) (layer B.Cu) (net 7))
 (segment (start 145.3166 55.9498) (end 145.3166 55.839798) (width 0.3) (layer B.Cu) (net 7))
 (segment (start 118.0846 41.3258) (end 118.0846 52.6818) (width 0.5) (layer B.Cu) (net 9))
 (segment (start 118.0846 52.6818) (end 116.8166 53.9498) (width 0.5) (layer B.Cu) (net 9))
 (segment (start 118.0846 38.7858) (end 118.0846 41.3258) (width 0.5) (layer B.Cu) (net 9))
 (segment (start 119.9666 53.9498) (end 118.8166 53.9498) (width 0.5) (layer B.Cu) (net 10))
 (segment (start 120.6246 41.3258) (end 120.6246 53.2918) (width 0.5) (layer B.Cu) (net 10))
 (segment (start 120.6246 53.2918) (end 119.9666 53.9498) (width 0.5) (layer B.Cu) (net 10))
 (segment (start 120.6246 38.7858) (end 120.6246 41.3258) (width 0.5) (layer B.Cu) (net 10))
 (segment (start 119.9388 57.5056) (end 117.2224 57.5056) (width 0.5) (layer B.Cu) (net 11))
 (segment (start 117.2224 57.5056) (end 116.8166 57.0998) (width 0.5) (layer B.Cu) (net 11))
 (segment (start 116.8166 57.0998) (end 116.8166 55.9498) (width 0.5) (layer B.Cu) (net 11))
 (segment (start 125.7046 51.7398) (end 119.9388 57.5056) (width 0.5) (layer B.Cu) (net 11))
 (segment (start 125.7046 41.3258) (end 125.7046 51.7398) (width 0.5) (layer B.Cu) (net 11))
 (segment (start 125.7046 38.7858) (end 125.7046 41.3258) (width 0.5) (layer B.Cu) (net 11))
 (segment (start 123.1646 52.7518) (end 119.9666 55.9498) (width 0.5) (layer B.Cu) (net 12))
 (segment (start 123.1646 41.3258) (end 123.1646 52.7518) (width 0.5) (layer B.Cu) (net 12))
 (segment (start 119.9666 55.9498) (end 118.8166 55.9498) (width 0.5) (layer B.Cu) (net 12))
 (segment (start 123.1646 38.7858) (end 123.1646 41.3258) (width 0.5) (layer B.Cu) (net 12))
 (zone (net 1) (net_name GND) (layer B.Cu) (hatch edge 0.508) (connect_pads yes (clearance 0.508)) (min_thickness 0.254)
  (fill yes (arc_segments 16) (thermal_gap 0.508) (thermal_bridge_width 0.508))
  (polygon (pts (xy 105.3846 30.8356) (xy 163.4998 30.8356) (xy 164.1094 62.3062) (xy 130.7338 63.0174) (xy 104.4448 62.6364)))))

